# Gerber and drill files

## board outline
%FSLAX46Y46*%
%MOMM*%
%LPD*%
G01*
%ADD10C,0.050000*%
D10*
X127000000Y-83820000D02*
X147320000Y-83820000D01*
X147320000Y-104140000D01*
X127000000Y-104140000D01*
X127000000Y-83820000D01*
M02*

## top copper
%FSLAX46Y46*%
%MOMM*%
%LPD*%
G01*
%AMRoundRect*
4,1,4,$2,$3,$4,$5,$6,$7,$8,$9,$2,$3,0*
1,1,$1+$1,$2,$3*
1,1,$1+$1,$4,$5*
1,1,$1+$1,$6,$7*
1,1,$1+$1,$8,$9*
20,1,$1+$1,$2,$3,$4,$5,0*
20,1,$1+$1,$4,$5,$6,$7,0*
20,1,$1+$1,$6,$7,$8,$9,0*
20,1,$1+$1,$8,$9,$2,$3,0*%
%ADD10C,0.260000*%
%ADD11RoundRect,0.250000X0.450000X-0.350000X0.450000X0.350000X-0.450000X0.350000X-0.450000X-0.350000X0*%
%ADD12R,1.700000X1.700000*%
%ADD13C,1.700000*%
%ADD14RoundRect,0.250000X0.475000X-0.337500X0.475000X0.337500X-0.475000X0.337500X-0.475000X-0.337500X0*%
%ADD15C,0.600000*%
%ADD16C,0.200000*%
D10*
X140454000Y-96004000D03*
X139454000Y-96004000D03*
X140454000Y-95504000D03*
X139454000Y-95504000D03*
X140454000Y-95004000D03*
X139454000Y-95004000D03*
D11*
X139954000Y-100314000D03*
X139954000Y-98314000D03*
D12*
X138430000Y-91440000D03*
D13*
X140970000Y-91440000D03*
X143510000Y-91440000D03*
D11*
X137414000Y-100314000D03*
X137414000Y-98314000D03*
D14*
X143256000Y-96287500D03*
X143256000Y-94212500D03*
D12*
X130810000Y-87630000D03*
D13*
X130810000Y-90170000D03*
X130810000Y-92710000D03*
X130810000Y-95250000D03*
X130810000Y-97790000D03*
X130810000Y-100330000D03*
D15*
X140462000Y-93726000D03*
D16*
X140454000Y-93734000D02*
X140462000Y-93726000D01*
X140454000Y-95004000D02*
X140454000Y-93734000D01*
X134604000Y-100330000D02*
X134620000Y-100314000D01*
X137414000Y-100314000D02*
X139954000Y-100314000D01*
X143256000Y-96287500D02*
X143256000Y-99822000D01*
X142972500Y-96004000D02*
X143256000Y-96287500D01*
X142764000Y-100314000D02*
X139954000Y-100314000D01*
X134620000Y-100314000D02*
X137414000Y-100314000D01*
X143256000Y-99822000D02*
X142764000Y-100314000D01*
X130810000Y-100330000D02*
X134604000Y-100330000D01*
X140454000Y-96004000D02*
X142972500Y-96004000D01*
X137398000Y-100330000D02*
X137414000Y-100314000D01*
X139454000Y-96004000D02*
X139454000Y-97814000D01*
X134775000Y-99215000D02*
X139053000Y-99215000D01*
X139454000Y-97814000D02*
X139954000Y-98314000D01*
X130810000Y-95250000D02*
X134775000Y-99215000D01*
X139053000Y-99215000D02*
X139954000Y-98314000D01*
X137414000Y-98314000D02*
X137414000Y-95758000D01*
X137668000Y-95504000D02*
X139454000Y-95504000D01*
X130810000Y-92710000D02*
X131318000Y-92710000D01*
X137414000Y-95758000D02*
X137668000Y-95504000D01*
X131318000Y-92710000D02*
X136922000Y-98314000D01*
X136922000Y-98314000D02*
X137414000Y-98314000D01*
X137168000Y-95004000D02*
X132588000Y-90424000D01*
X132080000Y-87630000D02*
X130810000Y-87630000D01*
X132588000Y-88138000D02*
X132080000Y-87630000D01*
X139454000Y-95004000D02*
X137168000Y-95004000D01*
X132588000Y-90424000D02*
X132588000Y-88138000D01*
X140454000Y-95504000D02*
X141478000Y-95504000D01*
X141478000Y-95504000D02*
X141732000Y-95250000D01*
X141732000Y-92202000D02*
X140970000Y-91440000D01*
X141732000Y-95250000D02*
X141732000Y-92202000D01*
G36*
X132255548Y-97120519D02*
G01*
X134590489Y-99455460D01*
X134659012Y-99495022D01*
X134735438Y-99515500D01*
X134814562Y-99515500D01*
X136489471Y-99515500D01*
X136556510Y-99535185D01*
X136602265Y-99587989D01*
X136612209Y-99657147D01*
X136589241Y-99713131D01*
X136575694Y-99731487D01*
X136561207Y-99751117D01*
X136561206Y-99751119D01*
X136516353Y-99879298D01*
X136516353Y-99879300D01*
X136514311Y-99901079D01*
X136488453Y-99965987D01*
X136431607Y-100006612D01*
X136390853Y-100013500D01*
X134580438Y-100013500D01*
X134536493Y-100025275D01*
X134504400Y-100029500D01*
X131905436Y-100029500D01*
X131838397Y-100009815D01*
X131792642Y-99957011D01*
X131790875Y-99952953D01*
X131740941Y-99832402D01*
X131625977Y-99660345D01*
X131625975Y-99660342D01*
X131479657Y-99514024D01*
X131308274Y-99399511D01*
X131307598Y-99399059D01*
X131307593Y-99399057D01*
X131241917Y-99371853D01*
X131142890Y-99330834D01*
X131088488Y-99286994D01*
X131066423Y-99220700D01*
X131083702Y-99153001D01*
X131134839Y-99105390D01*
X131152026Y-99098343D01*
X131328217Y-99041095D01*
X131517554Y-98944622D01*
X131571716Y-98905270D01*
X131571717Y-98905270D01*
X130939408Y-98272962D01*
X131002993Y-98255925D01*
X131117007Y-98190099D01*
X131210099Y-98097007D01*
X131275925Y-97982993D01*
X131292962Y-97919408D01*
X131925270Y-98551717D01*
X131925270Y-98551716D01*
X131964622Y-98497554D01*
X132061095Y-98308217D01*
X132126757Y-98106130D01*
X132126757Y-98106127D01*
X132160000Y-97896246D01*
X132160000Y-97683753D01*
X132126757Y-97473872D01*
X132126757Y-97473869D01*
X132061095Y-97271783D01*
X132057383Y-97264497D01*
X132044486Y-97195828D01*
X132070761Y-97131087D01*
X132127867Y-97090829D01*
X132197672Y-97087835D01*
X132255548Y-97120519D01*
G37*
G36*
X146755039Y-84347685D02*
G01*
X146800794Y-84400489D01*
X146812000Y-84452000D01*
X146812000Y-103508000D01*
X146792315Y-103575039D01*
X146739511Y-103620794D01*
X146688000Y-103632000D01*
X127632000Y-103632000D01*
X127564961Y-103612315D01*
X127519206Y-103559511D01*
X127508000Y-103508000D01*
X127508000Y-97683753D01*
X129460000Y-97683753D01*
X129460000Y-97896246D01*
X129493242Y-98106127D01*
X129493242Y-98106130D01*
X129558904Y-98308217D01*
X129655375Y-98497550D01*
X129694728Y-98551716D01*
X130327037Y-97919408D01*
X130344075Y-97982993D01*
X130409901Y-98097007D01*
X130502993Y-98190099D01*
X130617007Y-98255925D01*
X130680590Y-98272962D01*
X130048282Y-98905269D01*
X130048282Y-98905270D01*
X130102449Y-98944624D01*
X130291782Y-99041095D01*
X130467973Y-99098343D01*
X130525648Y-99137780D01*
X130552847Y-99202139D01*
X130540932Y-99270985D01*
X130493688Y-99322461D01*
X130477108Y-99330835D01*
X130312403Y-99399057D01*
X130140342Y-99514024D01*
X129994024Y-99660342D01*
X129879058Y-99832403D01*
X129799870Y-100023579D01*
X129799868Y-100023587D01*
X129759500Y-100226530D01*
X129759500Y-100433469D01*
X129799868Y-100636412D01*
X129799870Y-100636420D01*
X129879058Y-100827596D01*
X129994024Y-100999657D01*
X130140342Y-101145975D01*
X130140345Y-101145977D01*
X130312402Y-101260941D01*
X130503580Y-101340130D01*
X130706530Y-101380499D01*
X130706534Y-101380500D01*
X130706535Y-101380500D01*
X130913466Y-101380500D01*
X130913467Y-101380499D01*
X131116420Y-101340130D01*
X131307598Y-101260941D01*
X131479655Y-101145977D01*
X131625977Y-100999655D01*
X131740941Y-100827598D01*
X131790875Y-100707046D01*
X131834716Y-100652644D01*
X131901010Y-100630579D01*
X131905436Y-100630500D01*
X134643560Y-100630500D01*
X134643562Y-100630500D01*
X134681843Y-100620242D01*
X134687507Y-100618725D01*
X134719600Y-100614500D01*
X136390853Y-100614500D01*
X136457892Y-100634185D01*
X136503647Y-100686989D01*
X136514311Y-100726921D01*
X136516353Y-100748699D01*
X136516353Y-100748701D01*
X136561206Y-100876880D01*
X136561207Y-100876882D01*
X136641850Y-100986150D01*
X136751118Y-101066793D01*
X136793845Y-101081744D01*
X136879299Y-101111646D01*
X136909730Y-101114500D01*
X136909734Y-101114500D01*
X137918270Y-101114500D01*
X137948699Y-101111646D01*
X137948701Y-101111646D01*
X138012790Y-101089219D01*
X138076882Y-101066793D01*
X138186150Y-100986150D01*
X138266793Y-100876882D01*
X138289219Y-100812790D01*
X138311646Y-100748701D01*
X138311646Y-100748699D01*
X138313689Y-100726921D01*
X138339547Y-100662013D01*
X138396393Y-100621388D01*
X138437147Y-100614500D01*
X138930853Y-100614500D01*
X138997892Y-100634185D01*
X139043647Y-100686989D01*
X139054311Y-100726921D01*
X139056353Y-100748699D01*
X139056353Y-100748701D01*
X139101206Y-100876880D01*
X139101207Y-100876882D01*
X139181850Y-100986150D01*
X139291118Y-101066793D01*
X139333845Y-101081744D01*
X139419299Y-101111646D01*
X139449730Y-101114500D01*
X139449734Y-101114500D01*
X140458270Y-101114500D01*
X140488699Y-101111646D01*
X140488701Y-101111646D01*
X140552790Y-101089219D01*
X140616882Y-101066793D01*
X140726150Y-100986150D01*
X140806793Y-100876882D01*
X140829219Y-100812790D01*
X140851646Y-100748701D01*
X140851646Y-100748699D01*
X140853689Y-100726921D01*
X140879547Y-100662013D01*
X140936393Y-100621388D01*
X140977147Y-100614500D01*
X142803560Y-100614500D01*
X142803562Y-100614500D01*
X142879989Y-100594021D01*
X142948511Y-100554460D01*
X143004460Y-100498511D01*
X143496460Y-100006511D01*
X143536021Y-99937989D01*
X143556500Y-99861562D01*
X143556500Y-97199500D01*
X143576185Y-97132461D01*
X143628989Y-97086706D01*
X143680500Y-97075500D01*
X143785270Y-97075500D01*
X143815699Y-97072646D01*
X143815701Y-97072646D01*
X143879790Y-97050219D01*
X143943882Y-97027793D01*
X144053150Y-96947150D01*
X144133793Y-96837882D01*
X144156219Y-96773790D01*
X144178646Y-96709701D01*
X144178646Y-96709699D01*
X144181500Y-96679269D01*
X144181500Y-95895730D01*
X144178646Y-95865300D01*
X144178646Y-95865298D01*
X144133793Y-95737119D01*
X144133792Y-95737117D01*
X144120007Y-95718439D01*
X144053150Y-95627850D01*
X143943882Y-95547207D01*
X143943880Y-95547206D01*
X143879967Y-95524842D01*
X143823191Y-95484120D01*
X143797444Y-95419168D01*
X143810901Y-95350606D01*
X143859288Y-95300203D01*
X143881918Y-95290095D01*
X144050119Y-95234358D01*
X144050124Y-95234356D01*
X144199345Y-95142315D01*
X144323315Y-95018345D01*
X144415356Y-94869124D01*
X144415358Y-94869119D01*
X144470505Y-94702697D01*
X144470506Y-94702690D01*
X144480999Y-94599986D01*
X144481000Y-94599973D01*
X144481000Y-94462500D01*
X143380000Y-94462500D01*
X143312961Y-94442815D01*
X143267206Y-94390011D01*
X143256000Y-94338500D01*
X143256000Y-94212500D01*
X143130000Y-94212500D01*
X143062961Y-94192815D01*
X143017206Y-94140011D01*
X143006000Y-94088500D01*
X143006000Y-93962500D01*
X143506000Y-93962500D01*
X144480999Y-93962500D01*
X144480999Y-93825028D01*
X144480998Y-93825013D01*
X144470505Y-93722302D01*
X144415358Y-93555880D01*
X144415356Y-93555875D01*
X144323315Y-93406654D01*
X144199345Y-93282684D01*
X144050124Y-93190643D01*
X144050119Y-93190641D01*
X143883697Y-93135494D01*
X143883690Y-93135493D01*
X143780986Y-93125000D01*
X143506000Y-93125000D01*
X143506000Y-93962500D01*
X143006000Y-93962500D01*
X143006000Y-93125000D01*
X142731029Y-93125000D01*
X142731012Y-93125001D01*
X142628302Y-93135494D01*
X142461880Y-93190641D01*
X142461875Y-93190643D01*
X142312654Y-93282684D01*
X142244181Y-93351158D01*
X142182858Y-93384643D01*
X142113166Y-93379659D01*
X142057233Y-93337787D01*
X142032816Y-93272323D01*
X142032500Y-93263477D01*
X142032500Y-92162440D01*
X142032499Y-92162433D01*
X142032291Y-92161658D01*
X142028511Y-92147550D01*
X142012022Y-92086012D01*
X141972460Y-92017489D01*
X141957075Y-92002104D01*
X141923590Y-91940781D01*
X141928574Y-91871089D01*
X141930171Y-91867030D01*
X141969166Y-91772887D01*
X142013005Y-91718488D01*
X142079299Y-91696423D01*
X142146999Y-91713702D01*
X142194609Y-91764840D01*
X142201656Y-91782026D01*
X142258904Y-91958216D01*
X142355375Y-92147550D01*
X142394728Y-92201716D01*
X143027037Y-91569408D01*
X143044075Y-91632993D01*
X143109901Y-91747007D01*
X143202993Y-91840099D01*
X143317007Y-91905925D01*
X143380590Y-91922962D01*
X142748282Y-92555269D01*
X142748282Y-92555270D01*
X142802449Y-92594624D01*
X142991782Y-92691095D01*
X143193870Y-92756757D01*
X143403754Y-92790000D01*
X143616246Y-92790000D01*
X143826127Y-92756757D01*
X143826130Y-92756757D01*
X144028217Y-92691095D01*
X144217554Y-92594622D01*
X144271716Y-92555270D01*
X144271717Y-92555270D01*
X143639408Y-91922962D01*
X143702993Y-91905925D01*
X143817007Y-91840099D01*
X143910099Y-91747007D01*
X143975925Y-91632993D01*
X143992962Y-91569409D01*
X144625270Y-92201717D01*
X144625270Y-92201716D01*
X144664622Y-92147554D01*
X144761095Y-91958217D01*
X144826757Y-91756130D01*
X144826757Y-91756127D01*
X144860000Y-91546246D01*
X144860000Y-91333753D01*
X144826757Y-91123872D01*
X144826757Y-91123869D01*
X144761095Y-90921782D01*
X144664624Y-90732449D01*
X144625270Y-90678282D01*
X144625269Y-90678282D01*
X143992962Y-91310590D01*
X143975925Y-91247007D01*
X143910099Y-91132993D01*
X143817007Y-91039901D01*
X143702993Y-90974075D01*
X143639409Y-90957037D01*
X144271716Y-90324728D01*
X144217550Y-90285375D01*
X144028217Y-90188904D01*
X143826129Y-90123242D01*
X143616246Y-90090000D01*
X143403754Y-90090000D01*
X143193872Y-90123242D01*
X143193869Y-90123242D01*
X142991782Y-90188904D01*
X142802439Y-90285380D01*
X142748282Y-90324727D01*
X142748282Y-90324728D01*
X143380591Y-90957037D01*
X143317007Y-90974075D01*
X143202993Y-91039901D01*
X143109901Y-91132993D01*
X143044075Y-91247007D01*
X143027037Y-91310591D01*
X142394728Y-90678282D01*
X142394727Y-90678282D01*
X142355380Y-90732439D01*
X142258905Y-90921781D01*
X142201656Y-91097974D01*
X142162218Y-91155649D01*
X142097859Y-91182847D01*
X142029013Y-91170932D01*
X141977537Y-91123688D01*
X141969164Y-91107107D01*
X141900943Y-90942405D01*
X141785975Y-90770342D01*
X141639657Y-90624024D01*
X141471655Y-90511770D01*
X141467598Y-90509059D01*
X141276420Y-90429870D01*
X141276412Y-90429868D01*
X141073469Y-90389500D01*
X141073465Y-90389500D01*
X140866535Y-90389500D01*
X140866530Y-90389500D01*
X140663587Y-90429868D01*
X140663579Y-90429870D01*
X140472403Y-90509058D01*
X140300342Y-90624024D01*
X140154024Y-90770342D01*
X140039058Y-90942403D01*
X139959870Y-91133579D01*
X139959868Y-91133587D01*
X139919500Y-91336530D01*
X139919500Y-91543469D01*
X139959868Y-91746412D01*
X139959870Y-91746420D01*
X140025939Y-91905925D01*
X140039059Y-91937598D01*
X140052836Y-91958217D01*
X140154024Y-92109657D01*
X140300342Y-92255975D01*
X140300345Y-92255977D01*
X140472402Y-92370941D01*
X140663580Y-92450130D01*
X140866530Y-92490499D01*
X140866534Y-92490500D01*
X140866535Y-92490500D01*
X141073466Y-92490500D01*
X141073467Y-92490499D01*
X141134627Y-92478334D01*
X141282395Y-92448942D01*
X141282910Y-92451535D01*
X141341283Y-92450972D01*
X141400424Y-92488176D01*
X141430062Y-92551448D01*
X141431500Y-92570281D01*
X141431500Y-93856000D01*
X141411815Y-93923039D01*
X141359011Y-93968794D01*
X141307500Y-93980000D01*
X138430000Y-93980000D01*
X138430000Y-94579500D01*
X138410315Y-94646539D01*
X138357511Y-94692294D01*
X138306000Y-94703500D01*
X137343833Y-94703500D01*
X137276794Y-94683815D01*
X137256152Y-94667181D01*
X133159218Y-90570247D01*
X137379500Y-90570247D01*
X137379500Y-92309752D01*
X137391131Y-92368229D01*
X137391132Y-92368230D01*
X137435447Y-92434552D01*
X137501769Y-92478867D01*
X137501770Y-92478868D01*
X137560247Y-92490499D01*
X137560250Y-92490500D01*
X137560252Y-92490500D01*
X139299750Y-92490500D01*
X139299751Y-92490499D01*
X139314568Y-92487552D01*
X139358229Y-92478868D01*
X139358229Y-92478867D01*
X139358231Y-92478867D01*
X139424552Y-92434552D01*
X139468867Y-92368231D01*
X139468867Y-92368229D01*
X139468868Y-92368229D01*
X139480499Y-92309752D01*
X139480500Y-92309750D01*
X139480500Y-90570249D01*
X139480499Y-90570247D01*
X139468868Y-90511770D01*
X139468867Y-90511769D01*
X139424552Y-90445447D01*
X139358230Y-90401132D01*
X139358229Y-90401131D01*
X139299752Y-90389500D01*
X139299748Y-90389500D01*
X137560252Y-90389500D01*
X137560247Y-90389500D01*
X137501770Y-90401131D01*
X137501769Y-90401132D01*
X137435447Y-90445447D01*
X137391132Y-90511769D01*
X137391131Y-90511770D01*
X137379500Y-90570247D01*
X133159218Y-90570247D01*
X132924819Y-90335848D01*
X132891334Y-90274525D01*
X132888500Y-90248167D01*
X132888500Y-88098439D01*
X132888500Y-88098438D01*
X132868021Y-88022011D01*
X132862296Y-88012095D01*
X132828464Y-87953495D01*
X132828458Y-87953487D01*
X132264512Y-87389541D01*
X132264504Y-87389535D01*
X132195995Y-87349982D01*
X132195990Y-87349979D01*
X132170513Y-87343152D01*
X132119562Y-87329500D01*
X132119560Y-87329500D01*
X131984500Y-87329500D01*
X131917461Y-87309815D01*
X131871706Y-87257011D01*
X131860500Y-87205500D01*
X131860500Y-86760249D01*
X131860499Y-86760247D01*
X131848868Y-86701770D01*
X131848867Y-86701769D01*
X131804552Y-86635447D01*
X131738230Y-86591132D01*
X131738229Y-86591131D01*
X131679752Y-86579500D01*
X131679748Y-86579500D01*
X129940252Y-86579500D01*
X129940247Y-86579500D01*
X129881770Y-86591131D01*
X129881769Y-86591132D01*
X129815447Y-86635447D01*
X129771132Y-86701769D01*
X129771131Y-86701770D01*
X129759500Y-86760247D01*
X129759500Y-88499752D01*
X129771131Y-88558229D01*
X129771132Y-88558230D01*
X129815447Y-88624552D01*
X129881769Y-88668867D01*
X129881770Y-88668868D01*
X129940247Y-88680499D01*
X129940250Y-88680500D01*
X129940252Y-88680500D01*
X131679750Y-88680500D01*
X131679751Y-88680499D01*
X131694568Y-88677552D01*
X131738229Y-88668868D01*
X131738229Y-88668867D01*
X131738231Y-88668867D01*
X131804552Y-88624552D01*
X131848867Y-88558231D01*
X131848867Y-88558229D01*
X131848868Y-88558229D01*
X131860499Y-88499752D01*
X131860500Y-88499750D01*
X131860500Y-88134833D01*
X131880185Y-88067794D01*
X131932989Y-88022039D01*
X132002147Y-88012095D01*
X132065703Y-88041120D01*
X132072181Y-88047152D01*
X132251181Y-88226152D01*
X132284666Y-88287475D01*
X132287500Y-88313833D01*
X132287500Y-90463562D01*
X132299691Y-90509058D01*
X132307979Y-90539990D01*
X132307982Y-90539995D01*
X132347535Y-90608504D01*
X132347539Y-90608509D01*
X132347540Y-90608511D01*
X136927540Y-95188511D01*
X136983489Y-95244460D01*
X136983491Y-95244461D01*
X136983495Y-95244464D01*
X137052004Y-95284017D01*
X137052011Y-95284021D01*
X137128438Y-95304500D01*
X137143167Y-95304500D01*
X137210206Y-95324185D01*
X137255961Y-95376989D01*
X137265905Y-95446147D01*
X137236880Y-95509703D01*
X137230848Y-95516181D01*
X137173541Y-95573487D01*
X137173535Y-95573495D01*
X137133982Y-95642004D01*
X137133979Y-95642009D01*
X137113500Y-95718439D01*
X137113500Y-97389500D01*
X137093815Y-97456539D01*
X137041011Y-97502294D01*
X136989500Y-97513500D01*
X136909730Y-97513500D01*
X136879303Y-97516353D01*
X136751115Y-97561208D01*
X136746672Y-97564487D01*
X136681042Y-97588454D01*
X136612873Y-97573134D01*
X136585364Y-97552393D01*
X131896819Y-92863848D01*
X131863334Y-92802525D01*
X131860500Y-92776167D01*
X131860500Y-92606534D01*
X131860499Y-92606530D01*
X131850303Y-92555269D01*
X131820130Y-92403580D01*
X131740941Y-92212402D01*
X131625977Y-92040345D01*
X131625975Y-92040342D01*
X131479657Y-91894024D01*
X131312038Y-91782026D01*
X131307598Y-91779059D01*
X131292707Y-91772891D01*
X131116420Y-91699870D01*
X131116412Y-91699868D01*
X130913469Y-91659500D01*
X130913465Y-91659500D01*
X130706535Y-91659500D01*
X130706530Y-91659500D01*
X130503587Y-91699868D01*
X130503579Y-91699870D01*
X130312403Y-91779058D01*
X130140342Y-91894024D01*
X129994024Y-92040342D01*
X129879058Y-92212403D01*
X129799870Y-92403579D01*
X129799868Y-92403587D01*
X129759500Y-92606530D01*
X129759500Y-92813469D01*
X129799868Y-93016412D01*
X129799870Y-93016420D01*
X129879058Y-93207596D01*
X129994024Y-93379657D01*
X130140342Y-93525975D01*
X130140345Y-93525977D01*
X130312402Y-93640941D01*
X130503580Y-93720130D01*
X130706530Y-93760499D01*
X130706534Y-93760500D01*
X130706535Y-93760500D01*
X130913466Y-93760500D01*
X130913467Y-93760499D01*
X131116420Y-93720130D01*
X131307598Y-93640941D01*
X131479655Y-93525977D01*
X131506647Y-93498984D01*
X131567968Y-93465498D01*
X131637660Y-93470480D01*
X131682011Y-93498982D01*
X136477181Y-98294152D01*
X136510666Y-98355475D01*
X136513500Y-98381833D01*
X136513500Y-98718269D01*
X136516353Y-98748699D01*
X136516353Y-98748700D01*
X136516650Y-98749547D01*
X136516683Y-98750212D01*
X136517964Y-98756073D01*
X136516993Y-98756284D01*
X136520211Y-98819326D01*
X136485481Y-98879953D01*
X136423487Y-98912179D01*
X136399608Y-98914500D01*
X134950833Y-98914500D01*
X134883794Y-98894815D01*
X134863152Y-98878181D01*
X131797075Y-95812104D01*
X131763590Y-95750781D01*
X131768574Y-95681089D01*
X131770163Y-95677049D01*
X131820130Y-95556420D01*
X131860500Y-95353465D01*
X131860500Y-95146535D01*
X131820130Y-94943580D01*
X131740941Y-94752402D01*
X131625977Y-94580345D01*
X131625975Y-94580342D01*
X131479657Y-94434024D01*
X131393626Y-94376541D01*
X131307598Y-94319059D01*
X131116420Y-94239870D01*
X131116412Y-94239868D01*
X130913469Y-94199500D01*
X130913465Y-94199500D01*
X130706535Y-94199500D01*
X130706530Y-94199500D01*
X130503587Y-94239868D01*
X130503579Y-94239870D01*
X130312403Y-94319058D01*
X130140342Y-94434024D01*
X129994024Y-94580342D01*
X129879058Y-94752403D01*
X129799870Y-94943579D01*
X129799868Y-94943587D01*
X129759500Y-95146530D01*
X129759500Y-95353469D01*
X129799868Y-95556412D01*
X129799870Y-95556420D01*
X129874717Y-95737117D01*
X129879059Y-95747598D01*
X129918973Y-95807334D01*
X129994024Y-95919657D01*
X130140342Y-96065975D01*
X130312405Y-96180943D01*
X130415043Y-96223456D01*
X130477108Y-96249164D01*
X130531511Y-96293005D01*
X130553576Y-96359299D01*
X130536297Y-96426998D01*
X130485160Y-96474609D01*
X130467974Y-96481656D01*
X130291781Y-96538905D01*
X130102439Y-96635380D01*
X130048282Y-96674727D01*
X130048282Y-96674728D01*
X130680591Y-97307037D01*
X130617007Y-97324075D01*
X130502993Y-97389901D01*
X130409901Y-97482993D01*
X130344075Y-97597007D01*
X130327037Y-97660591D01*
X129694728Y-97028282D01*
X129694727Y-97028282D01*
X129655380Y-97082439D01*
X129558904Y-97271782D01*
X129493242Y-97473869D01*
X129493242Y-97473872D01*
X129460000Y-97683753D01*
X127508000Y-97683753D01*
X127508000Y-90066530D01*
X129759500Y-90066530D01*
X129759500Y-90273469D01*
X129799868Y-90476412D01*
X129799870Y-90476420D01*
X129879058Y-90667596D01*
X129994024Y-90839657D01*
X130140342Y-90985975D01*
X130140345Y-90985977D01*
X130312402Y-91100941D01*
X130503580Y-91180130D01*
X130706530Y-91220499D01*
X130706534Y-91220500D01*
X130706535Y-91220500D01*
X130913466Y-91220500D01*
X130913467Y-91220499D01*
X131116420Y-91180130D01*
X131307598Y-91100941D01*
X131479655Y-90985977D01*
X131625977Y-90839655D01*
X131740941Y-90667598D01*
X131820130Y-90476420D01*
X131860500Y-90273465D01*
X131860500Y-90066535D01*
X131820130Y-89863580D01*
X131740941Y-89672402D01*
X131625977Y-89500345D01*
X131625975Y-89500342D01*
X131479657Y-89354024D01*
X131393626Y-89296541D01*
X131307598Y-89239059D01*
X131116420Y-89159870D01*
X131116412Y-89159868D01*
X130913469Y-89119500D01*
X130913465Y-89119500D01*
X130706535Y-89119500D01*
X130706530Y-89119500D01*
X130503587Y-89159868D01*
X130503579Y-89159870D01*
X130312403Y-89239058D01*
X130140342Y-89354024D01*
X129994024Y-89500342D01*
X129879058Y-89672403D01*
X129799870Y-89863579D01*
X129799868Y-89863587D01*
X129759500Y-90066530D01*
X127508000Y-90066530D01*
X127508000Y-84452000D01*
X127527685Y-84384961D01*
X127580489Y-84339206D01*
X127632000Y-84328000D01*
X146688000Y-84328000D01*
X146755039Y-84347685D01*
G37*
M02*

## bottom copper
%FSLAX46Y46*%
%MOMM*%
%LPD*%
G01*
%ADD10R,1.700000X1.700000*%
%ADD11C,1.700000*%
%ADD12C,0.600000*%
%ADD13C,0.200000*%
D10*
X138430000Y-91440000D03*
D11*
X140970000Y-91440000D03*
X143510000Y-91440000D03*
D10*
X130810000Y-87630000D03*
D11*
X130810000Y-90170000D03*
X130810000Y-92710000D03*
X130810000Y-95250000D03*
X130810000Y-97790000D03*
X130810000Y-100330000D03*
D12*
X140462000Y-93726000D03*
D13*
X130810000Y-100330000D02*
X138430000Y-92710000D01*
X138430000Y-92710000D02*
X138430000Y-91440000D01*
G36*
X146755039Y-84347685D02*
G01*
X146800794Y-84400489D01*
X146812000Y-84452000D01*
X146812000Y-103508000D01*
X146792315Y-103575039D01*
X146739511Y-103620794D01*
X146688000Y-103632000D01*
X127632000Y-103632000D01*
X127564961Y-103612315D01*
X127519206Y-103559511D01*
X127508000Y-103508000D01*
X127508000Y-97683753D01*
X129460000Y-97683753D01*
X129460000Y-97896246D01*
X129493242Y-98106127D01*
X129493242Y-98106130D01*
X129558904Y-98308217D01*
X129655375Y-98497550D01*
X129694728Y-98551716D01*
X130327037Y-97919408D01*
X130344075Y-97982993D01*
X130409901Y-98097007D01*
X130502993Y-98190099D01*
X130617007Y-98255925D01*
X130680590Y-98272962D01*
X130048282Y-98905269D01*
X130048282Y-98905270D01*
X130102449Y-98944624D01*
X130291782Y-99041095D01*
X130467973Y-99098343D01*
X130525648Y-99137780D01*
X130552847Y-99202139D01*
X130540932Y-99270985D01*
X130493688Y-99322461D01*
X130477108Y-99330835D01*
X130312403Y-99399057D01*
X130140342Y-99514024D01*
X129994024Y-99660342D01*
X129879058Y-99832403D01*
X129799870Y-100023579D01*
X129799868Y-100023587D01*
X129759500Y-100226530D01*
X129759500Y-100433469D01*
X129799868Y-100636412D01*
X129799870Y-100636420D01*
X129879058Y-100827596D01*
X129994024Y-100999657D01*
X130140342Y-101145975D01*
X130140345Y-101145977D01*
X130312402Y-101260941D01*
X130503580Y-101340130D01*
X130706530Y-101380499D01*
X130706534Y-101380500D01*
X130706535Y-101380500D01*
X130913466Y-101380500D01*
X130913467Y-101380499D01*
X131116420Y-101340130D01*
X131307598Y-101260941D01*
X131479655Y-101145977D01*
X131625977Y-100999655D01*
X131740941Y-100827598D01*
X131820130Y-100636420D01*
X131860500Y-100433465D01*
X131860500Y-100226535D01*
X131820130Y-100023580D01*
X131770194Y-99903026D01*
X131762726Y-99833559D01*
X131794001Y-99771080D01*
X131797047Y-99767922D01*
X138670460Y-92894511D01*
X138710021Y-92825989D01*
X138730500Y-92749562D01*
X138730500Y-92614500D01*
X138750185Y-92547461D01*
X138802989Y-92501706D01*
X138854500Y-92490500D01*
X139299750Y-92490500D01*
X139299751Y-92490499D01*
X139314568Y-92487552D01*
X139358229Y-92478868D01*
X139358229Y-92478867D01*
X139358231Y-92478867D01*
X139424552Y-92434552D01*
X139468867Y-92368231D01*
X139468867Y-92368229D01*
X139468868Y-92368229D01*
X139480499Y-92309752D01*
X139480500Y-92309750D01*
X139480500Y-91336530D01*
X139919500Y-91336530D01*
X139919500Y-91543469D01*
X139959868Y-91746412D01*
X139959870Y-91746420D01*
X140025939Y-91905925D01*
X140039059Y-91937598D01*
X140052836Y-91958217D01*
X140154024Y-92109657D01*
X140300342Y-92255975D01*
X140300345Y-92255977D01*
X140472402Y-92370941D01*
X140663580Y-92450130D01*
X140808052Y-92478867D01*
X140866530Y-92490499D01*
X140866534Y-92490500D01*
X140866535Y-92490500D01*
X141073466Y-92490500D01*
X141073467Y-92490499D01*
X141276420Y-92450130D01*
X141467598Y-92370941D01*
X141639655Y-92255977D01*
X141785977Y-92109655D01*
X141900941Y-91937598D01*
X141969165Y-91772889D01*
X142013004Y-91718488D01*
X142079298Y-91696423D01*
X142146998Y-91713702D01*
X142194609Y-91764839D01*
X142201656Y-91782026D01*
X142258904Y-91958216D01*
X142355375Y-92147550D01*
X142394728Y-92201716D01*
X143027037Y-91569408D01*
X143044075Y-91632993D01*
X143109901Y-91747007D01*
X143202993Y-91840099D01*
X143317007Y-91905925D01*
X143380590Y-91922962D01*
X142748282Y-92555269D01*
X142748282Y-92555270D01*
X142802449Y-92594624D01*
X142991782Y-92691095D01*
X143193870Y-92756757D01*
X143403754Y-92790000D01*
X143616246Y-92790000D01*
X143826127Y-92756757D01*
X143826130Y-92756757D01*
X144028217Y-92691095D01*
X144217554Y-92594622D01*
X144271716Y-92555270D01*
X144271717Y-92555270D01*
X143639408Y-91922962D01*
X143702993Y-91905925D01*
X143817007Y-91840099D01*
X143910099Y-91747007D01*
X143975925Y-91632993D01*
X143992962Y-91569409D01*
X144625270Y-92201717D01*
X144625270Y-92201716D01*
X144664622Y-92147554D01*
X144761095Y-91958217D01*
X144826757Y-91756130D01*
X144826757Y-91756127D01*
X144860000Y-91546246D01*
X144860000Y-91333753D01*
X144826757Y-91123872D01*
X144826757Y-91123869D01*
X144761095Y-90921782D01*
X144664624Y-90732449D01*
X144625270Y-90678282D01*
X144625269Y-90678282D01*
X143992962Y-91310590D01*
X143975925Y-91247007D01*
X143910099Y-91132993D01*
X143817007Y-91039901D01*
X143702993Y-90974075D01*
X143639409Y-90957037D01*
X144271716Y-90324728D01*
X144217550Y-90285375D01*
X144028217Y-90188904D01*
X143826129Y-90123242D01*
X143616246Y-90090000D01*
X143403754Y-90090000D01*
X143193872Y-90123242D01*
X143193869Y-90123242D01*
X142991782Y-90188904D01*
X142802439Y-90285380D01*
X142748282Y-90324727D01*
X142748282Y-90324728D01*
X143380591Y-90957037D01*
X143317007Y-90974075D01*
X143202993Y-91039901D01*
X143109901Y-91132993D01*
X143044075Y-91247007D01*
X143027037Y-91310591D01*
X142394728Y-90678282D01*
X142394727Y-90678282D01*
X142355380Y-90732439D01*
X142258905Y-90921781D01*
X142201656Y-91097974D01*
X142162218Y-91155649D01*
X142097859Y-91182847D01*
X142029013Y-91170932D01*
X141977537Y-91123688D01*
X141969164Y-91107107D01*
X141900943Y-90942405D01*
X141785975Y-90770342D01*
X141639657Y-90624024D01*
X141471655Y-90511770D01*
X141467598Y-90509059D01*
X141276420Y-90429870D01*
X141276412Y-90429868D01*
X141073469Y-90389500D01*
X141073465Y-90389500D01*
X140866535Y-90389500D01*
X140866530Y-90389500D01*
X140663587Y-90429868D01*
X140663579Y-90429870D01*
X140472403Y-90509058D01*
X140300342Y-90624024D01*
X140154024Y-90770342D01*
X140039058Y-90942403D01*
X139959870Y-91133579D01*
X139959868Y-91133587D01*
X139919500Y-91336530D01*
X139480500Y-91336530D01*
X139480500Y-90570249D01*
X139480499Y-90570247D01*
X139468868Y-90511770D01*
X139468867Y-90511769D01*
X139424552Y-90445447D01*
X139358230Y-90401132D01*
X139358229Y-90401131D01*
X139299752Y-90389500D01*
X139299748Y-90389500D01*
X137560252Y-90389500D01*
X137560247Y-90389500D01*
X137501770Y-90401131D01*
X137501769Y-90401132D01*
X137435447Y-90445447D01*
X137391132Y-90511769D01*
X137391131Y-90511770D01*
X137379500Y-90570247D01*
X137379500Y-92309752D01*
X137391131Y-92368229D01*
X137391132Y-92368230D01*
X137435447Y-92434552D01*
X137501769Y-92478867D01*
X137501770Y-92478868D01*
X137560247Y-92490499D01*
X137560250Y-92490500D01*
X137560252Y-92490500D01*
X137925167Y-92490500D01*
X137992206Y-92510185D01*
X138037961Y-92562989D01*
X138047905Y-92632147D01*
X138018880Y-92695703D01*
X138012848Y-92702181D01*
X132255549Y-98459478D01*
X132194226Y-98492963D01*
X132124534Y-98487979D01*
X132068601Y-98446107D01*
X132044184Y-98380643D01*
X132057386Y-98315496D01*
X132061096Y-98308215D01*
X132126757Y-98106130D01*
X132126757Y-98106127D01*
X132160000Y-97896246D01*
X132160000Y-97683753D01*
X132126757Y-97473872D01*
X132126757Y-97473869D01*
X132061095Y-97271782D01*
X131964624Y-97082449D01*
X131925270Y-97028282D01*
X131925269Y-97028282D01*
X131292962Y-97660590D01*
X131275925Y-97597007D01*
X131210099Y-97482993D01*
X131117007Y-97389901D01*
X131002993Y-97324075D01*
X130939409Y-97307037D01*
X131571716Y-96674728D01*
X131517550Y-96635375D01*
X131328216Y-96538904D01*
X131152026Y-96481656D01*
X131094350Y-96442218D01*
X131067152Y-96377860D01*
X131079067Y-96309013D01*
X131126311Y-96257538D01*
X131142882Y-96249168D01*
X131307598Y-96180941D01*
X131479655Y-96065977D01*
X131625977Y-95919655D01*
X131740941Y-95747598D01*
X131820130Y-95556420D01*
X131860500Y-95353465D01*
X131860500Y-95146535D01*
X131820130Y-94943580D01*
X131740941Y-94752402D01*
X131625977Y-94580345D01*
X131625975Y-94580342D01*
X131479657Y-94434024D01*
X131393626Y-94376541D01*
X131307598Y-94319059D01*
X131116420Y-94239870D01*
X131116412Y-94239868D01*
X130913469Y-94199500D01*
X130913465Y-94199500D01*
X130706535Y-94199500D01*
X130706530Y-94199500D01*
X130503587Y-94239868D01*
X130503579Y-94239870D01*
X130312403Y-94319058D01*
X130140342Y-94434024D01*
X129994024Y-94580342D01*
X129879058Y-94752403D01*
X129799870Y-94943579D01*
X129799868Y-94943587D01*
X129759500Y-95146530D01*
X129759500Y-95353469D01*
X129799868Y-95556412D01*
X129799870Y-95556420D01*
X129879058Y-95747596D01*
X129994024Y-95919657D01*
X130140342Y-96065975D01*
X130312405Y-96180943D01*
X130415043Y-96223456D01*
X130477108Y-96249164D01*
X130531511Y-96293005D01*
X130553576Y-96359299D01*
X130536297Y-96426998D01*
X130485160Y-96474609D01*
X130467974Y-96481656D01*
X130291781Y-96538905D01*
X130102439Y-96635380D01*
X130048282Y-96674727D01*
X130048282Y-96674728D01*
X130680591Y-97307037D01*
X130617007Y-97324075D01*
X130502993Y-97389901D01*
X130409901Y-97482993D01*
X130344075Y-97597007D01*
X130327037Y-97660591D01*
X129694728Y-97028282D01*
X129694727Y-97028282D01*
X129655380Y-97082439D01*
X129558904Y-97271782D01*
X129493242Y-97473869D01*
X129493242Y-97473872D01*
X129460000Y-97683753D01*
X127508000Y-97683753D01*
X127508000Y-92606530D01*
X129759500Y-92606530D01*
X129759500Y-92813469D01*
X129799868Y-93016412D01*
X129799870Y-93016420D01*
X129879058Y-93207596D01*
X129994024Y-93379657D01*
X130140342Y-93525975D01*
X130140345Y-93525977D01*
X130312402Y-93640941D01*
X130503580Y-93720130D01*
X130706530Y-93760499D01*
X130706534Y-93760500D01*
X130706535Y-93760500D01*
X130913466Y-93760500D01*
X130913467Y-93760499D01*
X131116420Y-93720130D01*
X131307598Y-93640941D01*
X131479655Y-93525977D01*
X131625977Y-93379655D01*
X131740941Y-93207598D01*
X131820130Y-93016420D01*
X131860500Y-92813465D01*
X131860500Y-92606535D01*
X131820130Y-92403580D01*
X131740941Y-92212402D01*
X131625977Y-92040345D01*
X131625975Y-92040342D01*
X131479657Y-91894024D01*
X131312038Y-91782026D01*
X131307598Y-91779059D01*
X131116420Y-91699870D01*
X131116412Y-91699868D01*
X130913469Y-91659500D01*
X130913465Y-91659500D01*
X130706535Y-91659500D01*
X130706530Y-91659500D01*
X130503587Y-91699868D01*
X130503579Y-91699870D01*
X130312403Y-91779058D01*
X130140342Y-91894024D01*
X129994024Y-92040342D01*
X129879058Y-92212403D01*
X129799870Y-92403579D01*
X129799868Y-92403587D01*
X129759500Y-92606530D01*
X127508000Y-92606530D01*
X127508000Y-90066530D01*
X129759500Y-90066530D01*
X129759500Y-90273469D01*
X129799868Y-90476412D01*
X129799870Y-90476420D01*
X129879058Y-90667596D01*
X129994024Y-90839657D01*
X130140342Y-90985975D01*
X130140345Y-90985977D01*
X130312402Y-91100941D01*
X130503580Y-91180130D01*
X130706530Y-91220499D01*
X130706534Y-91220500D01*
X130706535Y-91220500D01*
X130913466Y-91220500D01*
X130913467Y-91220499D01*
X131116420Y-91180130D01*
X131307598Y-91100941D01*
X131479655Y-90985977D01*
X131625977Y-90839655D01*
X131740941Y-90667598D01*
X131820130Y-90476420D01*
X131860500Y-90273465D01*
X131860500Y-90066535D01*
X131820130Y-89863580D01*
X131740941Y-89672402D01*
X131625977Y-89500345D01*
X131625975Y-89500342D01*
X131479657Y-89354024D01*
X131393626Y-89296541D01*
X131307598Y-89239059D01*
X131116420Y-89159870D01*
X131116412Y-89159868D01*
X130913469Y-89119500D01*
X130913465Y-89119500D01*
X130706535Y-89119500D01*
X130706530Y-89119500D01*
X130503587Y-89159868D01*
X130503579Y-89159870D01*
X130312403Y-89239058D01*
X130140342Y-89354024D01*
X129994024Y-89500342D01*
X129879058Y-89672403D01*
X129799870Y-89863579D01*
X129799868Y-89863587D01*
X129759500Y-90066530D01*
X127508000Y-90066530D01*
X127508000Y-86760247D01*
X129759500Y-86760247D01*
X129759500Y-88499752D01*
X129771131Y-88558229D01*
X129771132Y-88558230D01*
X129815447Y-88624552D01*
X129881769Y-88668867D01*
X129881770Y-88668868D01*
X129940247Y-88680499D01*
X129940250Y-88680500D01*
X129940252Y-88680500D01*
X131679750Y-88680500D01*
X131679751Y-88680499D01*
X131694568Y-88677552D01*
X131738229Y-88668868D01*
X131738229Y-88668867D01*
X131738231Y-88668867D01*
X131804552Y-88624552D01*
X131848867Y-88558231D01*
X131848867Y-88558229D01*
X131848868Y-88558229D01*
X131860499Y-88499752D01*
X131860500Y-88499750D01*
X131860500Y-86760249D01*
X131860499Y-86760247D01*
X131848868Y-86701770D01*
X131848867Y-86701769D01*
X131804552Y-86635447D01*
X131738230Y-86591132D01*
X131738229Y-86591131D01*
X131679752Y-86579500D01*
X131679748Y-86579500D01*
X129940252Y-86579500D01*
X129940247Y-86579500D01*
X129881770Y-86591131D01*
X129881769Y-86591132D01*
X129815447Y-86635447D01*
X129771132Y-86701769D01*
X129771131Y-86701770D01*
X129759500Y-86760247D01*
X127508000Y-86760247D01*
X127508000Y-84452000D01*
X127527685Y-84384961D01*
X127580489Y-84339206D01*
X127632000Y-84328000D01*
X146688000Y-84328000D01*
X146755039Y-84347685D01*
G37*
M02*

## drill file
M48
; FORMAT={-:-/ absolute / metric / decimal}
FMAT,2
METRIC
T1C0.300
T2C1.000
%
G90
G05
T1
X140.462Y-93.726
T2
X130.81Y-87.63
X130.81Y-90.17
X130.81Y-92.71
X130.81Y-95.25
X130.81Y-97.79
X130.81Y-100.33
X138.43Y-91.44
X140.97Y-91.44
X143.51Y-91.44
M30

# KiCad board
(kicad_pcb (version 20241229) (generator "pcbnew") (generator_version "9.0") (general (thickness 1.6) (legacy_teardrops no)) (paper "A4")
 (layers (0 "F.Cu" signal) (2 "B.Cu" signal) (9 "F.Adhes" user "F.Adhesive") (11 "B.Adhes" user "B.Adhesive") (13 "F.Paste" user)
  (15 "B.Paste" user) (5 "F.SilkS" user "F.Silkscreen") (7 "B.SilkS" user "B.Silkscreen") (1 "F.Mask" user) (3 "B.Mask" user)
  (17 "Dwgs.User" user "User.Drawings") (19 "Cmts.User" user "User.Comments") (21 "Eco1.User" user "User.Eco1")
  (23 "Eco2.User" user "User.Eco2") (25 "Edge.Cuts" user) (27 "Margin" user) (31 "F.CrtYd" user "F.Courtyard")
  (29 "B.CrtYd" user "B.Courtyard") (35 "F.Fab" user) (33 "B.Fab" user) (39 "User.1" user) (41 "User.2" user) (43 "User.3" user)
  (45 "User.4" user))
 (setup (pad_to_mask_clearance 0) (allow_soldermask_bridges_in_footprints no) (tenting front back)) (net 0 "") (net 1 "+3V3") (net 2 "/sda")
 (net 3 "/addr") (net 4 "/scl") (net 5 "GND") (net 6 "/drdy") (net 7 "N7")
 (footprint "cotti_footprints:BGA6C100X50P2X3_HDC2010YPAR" (layer "F.Cu") (at 139.954 95.504 180)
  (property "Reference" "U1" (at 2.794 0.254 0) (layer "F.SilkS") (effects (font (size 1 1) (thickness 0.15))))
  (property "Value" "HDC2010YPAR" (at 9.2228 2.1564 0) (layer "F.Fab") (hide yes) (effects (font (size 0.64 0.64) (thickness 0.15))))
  (pad "A1" smd circle (at -0.5 -0.5 180) (size 0.26 0.26) (layers "F.Cu" "F.Mask" "F.Paste") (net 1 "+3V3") (solder_mask_margin 0.102))
  (pad "A2" smd circle (at 0.5 -0.5 180) (size 0.26 0.26) (layers "F.Cu" "F.Mask" "F.Paste") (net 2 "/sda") (solder_mask_margin 0.102))
  (pad "B1" smd circle (at -0.5 0 180) (size 0.26 0.26) (layers "F.Cu" "F.Mask" "F.Paste") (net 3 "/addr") (solder_mask_margin 0.102))
  (pad "B2" smd circle (at 0.5 0 180) (size 0.26 0.26) (layers "F.Cu" "F.Mask" "F.Paste") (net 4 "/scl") (solder_mask_margin 0.102))
  (pad "C1" smd circle (at -0.5 0.5 180) (size 0.26 0.26) (layers "F.Cu" "F.Mask" "F.Paste") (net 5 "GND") (solder_mask_margin 0.102))
  (pad "C2" smd circle (at 0.5 0.5 180) (size 0.26 0.26) (layers "F.Cu" "F.Mask" "F.Paste") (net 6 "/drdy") (solder_mask_margin 0.102)))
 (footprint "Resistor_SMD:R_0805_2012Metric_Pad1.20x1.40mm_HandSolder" (layer "F.Cu") (at 139.954 99.314 90)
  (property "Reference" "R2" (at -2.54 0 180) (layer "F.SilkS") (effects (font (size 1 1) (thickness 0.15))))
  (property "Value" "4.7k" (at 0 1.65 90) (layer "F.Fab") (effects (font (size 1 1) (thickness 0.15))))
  (pad "1" smd roundrect (at -1 0 90) (size 1.2 1.4) (layers "F.Cu" "F.Mask" "F.Paste") (roundrect_rratio 0.208333) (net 1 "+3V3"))
  (pad "2" smd roundrect (at 1 0 90) (size 1.2 1.4) (layers "F.Cu" "F.Mask" "F.Paste") (roundrect_rratio 0.208333) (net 2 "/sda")))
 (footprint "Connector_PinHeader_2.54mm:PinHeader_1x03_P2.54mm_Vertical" (layer "F.Cu") (at 138.43 91.44 90)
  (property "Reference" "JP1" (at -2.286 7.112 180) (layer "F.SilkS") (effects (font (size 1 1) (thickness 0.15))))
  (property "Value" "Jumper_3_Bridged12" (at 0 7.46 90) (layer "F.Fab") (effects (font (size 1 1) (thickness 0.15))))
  (pad "1" thru_hole rect (at 0 0 90) (size 1.7 1.7) (drill 1) (layers "*.Cu" "*.Mask") (remove_unused_layers no) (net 1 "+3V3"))
  (pad "2" thru_hole circle (at 0 2.54 90) (size 1.7 1.7) (drill 1) (layers "*.Cu" "*.Mask") (remove_unused_layers no) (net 3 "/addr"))
  (pad "3" thru_hole circle (at 0 5.08 90) (size 1.7 1.7) (drill 1) (layers "*.Cu" "*.Mask") (remove_unused_layers no) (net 5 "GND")))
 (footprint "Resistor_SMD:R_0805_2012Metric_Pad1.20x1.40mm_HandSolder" (layer "F.Cu") (at 137.414 99.314 90)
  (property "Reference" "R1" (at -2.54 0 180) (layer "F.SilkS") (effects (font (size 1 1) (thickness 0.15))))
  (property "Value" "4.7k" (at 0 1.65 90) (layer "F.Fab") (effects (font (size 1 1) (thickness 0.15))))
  (pad "1" smd roundrect (at -1 0 90) (size 1.2 1.4) (layers "F.Cu" "F.Mask" "F.Paste") (roundrect_rratio 0.208333) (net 1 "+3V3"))
  (pad "2" smd roundrect (at 1 0 90) (size 1.2 1.4) (layers "F.Cu" "F.Mask" "F.Paste") (roundrect_rratio 0.208333) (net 4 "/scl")))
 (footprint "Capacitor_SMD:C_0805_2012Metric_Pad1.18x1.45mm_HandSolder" (layer "F.Cu") (at 143.256 95.25 90)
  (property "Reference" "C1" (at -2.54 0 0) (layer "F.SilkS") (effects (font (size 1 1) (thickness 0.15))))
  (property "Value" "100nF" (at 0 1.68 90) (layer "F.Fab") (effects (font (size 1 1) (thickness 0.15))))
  (pad "1" smd roundrect (at -1.0375 0 90) (size 1.175 1.45) (layers "F.Cu" "F.Mask" "F.Paste") (roundrect_rratio 0.212766) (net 1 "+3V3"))
  (pad "2" smd roundrect (at 1.0375 0 90) (size 1.175 1.45) (layers "F.Cu" "F.Mask" "F.Paste") (roundrect_rratio 0.212766) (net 5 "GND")))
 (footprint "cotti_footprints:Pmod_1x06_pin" (layer "F.Cu") (at 130.81 87.63)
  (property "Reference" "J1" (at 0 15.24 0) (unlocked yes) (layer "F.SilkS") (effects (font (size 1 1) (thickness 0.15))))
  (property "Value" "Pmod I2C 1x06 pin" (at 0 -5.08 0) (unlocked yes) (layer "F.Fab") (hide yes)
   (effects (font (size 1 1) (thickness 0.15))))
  (pad "1" thru_hole rect (at 0 0) (size 1.7 1.7) (drill 1) (layers "*.Cu" "*.Mask") (remove_unused_layers no) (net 6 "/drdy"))
  (pad "2" thru_hole circle (at 0 2.54) (size 1.7 1.7) (drill 1) (layers "*.Cu" "*.Mask") (remove_unused_layers no) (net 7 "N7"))
  (pad "3" thru_hole circle (at 0 5.08) (size 1.7 1.7) (drill 1) (layers "*.Cu" "*.Mask") (remove_unused_layers no) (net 4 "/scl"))
  (pad "4" thru_hole circle (at 0 7.62) (size 1.7 1.7) (drill 1) (layers "*.Cu" "*.Mask") (remove_unused_layers no) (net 2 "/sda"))
  (pad "5" thru_hole circle (at 0 10.16) (size 1.7 1.7) (drill 1) (layers "*.Cu" "*.Mask") (remove_unused_layers no) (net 5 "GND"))
  (pad "6" thru_hole circle (at 0 12.7) (size 1.7 1.7) (drill 1) (layers "*.Cu" "*.Mask") (remove_unused_layers no) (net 1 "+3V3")))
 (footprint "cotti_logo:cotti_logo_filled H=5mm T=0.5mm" (layer "B.Cu") (at 143.427851 97.693 180)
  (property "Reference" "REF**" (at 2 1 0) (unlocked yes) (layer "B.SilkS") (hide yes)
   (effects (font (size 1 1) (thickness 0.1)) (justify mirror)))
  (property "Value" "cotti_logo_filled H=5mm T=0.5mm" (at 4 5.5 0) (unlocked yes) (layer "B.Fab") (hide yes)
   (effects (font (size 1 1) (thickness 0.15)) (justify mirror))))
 (gr_rect (start 127 83.82) (end 147.32 104.14) (stroke (width 0.05) (type default)) (fill no) (layer "Edge.Cuts"))
 (segment (start 140.454 93.734) (end 140.462 93.726) (width 0.2) (layer "F.Cu") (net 5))
 (segment (start 140.454 95.004) (end 140.454 93.734) (width 0.2) (layer "F.Cu") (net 5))
 (via (at 140.462 93.726) (size 0.6) (drill 0.3) (layers "F.Cu" "B.Cu") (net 5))
 (segment (start 134.604 100.33) (end 134.62 100.314) (width 0.2) (layer "F.Cu") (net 1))
 (segment (start 137.414 100.314) (end 139.954 100.314) (width 0.2) (layer "F.Cu") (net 1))
 (segment (start 143.256 96.2875) (end 143.256 99.822) (width 0.2) (layer "F.Cu") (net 1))
 (segment (start 142.9725 96.004) (end 143.256 96.2875) (width 0.2) (layer "F.Cu") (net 1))
 (segment (start 142.764 100.314) (end 139.954 100.314) (width 0.2) (layer "F.Cu") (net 1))
 (segment (start 134.62 100.314) (end 137.414 100.314) (width 0.2) (layer "F.Cu") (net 1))
 (segment (start 143.256 99.822) (end 142.764 100.314) (width 0.2) (layer "F.Cu") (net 1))
 (segment (start 130.81 100.33) (end 134.604 100.33) (width 0.2) (layer "F.Cu") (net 1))
 (segment (start 140.454 96.004) (end 142.9725 96.004) (width 0.2) (layer "F.Cu") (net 1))
 (segment (start 137.398 100.33) (end 137.414 100.314) (width 0.2) (layer "F.Cu") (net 1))
 (segment (start 130.81 100.33) (end 138.43 92.71) (width 0.2) (layer "B.Cu") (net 1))
 (segment (start 138.43 92.71) (end 138.43 91.44) (width 0.2) (layer "B.Cu") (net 1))
 (segment (start 139.454 96.004) (end 139.454 97.814) (width 0.2) (layer "F.Cu") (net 2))
 (segment (start 134.775 99.215) (end 139.053 99.215) (width 0.2) (layer "F.Cu") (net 2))
 (segment (start 139.454 97.814) (end 139.954 98.314) (width 0.2) (layer "F.Cu") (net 2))
 (segment (start 130.81 95.25) (end 134.775 99.215) (width 0.2) (layer "F.Cu") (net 2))
 (segment (start 139.053 99.215) (end 139.954 98.314) (width 0.2) (layer "F.Cu") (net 2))
 (segment (start 137.414 98.314) (end 137.414 95.758) (width 0.2) (layer "F.Cu") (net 4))
 (segment (start 137.668 95.504) (end 139.454 95.504) (width 0.2) (layer "F.Cu") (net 4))
 (segment (start 130.81 92.71) (end 131.318 92.71) (width 0.2) (layer "F.Cu") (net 4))
 (segment (start 137.414 95.758) (end 137.668 95.504) (width 0.2) (layer "F.Cu") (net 4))
 (segment (start 131.318 92.71) (end 136.922 98.314) (width 0.2) (layer "F.Cu") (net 4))
 (segment (start 136.922 98.314) (end 137.414 98.314) (width 0.2) (layer "F.Cu") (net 4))
 (segment (start 137.168 95.004) (end 132.588 90.424) (width 0.2) (layer "F.Cu") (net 6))
 (segment (start 132.08 87.63) (end 130.81 87.63) (width 0.2) (layer "F.Cu") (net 6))
 (segment (start 132.588 88.138) (end 132.08 87.63) (width 0.2) (layer "F.Cu") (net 6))
 (segment (start 139.454 95.004) (end 137.168 95.004) (width 0.2) (layer "F.Cu") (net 6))
 (segment (start 132.588 90.424) (end 132.588 88.138) (width 0.2) (layer "F.Cu") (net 6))
 (segment (start 140.454 95.504) (end 141.478 95.504) (width 0.2) (layer "F.Cu") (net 3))
 (segment (start 141.478 95.504) (end 141.732 95.25) (width 0.2) (layer "F.Cu") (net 3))
 (segment (start 141.732 92.202) (end 140.97 91.44) (width 0.2) (layer "F.Cu") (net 3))
 (segment (start 141.732 95.25) (end 141.732 92.202) (width 0.2) (layer "F.Cu") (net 3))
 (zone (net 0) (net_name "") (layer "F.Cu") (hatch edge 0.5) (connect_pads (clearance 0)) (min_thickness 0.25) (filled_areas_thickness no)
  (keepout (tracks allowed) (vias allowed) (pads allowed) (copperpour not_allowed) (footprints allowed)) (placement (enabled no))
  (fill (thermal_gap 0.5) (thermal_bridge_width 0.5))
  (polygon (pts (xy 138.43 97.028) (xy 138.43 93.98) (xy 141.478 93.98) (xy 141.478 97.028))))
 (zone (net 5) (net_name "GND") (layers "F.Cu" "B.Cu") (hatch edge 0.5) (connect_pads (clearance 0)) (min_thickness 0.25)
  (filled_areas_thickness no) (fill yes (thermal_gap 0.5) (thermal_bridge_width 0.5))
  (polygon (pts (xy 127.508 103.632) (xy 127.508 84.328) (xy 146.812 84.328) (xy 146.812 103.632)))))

